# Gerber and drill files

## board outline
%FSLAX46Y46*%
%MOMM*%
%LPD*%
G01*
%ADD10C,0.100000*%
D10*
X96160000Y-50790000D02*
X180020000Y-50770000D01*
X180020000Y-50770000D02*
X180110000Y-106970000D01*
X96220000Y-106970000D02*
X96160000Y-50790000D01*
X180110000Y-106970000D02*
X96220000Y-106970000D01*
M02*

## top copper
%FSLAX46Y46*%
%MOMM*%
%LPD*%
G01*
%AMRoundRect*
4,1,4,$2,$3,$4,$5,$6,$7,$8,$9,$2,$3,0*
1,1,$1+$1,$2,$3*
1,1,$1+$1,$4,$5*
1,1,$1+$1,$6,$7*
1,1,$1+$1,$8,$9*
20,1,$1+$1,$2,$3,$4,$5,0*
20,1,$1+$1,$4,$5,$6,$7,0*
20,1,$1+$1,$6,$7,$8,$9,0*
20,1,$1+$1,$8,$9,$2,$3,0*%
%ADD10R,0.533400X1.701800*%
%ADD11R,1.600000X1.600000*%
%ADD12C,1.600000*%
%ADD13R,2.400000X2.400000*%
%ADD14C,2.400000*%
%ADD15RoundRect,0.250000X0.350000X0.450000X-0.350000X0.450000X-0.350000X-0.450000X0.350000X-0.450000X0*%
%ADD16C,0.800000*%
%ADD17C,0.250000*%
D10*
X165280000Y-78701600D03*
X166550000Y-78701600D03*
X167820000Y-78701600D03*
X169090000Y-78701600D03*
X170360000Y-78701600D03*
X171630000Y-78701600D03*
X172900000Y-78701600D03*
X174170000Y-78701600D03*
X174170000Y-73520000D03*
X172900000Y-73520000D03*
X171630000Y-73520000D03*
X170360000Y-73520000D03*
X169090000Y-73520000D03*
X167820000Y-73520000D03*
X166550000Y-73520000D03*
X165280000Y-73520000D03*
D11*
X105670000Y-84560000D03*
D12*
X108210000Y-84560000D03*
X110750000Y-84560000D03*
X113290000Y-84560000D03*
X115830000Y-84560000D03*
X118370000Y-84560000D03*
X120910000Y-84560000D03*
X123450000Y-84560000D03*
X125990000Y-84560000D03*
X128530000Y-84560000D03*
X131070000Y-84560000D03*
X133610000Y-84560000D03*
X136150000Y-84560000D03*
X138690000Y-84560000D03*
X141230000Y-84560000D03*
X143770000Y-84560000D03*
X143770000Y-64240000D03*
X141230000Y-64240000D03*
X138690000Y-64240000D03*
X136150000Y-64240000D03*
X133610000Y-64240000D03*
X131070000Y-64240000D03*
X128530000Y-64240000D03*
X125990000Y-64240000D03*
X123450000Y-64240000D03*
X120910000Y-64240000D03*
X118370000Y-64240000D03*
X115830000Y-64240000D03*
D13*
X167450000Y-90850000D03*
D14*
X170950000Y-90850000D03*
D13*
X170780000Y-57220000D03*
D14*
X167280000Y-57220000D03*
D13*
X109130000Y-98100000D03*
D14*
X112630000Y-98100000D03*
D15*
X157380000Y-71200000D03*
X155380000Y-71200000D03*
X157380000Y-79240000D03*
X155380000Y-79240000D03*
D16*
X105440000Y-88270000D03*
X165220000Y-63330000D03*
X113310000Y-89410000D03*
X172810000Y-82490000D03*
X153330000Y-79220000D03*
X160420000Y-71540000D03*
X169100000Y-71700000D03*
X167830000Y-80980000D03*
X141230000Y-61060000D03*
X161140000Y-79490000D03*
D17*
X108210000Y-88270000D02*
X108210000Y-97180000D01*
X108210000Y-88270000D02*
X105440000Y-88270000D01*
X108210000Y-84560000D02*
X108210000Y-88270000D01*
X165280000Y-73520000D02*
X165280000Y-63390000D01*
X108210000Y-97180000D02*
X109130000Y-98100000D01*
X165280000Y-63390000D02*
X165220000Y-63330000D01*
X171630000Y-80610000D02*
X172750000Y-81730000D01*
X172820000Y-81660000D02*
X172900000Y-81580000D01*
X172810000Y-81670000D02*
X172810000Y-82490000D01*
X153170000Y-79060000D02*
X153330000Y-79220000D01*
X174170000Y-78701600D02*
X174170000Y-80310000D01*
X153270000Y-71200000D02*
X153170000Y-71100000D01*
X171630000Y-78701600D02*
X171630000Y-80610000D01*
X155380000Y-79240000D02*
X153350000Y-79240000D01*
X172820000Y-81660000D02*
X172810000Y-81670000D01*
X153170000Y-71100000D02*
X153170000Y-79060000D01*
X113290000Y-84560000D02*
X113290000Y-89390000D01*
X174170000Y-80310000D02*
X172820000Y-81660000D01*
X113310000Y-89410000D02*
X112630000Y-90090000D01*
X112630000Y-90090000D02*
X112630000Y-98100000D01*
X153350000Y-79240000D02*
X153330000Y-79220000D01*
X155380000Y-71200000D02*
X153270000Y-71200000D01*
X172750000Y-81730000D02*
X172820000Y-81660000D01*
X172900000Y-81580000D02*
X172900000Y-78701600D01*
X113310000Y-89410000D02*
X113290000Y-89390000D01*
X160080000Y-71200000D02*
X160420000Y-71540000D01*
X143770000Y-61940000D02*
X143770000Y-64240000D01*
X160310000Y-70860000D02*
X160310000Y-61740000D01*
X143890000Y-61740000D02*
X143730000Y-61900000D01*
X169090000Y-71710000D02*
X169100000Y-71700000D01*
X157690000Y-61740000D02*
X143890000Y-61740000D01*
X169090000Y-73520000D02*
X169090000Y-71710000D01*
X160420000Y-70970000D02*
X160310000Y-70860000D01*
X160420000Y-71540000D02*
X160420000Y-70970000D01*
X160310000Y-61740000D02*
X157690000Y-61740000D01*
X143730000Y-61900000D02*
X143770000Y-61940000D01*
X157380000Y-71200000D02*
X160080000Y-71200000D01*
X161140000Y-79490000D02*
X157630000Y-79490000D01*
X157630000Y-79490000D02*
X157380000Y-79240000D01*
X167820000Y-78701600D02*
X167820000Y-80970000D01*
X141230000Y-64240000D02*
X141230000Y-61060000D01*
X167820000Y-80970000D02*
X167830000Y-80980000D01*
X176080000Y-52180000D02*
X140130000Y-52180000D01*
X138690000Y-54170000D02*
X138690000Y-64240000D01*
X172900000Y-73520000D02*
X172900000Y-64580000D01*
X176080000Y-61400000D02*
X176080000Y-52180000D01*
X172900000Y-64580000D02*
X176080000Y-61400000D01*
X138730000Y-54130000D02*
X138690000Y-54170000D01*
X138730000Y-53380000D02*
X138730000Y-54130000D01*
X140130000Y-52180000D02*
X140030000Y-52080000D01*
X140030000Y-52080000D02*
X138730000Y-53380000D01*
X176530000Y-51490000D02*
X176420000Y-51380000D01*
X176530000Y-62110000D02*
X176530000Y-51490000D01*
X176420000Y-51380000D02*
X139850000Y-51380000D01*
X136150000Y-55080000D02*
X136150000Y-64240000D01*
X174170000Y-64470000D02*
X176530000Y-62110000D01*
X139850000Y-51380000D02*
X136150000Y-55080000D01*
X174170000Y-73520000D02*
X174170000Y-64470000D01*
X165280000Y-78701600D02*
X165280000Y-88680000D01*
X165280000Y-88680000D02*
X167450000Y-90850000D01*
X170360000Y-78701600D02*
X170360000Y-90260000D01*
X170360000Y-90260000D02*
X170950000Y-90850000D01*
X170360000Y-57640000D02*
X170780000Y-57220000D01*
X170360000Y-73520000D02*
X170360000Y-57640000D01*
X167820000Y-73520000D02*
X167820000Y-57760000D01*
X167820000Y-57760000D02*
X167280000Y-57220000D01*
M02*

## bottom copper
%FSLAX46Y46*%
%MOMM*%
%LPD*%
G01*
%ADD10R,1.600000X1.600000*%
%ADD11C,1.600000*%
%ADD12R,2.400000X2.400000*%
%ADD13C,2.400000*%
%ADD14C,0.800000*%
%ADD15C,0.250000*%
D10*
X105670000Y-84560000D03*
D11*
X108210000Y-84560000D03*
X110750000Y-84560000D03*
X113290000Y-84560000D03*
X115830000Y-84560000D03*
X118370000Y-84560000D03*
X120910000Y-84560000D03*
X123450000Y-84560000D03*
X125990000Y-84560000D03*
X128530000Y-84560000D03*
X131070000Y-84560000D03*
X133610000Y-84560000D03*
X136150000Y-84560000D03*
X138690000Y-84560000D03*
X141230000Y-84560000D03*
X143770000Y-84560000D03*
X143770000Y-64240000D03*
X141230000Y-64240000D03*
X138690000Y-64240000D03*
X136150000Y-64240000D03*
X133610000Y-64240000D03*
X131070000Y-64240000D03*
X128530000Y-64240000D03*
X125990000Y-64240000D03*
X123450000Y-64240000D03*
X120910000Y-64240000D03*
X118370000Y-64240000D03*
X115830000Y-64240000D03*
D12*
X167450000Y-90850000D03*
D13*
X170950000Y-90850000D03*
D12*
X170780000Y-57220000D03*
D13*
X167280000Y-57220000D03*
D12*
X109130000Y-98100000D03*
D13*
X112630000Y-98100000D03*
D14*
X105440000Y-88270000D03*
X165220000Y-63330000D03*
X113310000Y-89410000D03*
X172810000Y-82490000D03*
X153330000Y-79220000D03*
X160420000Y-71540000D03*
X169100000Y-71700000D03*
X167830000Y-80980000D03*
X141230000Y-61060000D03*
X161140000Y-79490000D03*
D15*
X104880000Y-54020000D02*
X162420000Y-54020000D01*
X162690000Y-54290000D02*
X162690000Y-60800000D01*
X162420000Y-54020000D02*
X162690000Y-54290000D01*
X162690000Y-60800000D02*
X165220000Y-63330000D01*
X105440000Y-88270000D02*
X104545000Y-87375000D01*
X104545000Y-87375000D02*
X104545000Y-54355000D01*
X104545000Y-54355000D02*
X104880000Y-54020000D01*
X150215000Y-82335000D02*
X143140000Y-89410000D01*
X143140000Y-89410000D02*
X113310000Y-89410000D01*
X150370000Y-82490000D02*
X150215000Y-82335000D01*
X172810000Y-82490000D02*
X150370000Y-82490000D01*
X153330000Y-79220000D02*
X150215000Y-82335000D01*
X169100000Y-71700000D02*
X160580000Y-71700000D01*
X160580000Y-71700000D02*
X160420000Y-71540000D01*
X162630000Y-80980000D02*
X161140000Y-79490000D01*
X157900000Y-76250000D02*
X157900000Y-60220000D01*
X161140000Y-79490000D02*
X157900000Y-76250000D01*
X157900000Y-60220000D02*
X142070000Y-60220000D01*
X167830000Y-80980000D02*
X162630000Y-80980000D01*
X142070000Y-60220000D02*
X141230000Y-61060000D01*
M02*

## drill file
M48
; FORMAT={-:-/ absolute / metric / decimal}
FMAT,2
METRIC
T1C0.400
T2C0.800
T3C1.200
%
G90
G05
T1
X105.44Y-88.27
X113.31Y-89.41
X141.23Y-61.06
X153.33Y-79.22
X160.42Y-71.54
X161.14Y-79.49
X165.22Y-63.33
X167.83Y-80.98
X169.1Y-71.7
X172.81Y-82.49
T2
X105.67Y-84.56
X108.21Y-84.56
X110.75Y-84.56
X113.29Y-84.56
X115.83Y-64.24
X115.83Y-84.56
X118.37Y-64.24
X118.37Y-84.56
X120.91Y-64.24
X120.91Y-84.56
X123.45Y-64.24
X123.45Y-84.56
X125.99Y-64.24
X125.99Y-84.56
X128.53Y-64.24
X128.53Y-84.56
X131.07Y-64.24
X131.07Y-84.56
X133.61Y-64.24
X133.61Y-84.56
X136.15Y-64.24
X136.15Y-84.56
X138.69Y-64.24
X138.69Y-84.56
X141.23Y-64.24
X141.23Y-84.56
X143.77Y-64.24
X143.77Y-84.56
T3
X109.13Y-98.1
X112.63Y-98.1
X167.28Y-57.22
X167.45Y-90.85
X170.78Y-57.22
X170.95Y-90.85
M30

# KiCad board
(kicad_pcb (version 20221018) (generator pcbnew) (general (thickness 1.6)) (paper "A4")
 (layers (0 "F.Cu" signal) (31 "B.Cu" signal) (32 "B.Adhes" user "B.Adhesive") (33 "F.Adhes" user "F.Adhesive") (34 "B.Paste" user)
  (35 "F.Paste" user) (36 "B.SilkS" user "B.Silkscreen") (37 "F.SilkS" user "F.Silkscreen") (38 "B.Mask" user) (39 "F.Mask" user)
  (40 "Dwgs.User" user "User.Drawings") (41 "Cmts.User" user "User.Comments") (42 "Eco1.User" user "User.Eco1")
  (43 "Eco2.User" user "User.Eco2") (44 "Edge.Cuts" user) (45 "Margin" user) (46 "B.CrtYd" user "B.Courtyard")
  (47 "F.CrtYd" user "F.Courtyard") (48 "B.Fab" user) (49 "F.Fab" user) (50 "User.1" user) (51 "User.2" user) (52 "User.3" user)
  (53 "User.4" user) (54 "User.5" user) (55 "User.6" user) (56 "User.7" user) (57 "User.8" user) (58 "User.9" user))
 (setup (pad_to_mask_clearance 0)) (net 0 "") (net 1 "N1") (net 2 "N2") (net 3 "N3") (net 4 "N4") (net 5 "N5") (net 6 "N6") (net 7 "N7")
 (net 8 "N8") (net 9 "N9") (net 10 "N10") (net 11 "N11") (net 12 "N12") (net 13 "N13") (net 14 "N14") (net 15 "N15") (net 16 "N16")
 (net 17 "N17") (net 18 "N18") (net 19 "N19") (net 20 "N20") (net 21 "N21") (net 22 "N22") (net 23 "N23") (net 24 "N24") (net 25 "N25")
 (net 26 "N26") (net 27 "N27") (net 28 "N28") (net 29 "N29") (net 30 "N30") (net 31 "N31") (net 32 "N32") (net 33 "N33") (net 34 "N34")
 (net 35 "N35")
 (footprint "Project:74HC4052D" (layer "F.Cu") (at 169.725 76.1108 90)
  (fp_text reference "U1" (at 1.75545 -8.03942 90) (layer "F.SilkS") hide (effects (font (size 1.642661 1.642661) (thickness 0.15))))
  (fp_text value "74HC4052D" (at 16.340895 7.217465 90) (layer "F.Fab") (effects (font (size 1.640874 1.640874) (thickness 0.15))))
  (pad "1" smd rect (at -2.5908 -4.445 90) (size 1.7018 0.5334) (layers "F.Cu" "F.Paste" "F.Mask") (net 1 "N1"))
  (pad "2" smd rect (at -2.5908 -3.175 90) (size 1.7018 0.5334) (layers "F.Cu" "F.Paste" "F.Mask") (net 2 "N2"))
  (pad "3" smd rect (at -2.5908 -1.905 90) (size 1.7018 0.5334) (layers "F.Cu" "F.Paste" "F.Mask") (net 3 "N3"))
  (pad "4" smd rect (at -2.5908 -0.635 90) (size 1.7018 0.5334) (layers "F.Cu" "F.Paste" "F.Mask") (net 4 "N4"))
  (pad "5" smd rect (at -2.5908 0.635 90) (size 1.7018 0.5334) (layers "F.Cu" "F.Paste" "F.Mask") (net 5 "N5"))
  (pad "6" smd rect (at -2.5908 1.905 90) (size 1.7018 0.5334) (layers "F.Cu" "F.Paste" "F.Mask") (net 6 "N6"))
  (pad "7" smd rect (at -2.5908 3.175 90) (size 1.7018 0.5334) (layers "F.Cu" "F.Paste" "F.Mask") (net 6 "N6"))
  (pad "8" smd rect (at -2.5908 4.445 90) (size 1.7018 0.5334) (layers "F.Cu" "F.Paste" "F.Mask") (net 6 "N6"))
  (pad "9" smd rect (at 2.5908 4.445 90) (size 1.7018 0.5334) (layers "F.Cu" "F.Paste" "F.Mask") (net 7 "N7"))
  (pad "10" smd rect (at 2.5908 3.175 90) (size 1.7018 0.5334) (layers "F.Cu" "F.Paste" "F.Mask") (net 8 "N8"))
  (pad "11" smd rect (at 2.5908 1.905 90) (size 1.7018 0.5334) (layers "F.Cu" "F.Paste" "F.Mask") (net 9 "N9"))
  (pad "12" smd rect (at 2.5908 0.635 90) (size 1.7018 0.5334) (layers "F.Cu" "F.Paste" "F.Mask") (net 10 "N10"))
  (pad "13" smd rect (at 2.5908 -0.635 90) (size 1.7018 0.5334) (layers "F.Cu" "F.Paste" "F.Mask") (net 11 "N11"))
  (pad "14" smd rect (at 2.5908 -1.905 90) (size 1.7018 0.5334) (layers "F.Cu" "F.Paste" "F.Mask") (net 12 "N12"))
  (pad "15" smd rect (at 2.5908 -3.175 90) (size 1.7018 0.5334) (layers "F.Cu" "F.Paste" "F.Mask") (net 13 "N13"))
  (pad "16" smd rect (at 2.5908 -4.445 90) (size 1.7018 0.5334) (layers "F.Cu" "F.Paste" "F.Mask") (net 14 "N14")))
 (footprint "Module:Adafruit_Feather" (layer "F.Cu") (at 105.67 84.56 90)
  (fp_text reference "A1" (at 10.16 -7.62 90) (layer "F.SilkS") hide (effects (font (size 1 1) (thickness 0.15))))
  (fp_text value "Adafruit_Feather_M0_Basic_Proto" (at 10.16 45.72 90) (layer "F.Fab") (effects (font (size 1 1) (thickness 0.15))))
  (pad "1" thru_hole rect (at 0 0 270) (size 1.6 1.6) (drill 0.8) (layers "*.Cu" "*.Mask") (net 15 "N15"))
  (pad "2" thru_hole circle (at 0 2.54 270) (size 1.6 1.6) (drill 0.8) (layers "*.Cu" "*.Mask") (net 14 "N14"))
  (pad "3" thru_hole circle (at 0 5.08 270) (size 1.6 1.6) (drill 0.8) (layers "*.Cu" "*.Mask") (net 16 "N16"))
  (pad "4" thru_hole circle (at 0 7.62 270) (size 1.6 1.6) (drill 0.8) (layers "*.Cu" "*.Mask") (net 6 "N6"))
  (pad "5" thru_hole circle (at 0 10.16 270) (size 1.6 1.6) (drill 0.8) (layers "*.Cu" "*.Mask") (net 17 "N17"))
  (pad "6" thru_hole circle (at 0 12.7 270) (size 1.6 1.6) (drill 0.8) (layers "*.Cu" "*.Mask") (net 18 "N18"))
  (pad "7" thru_hole circle (at 0 15.24 270) (size 1.6 1.6) (drill 0.8) (layers "*.Cu" "*.Mask") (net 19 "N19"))
  (pad "8" thru_hole circle (at 0 17.78 270) (size 1.6 1.6) (drill 0.8) (layers "*.Cu" "*.Mask") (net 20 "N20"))
  (pad "9" thru_hole circle (at 0 20.32 270) (size 1.6 1.6) (drill 0.8) (layers "*.Cu" "*.Mask") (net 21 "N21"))
  (pad "10" thru_hole circle (at 0 22.86 270) (size 1.6 1.6) (drill 0.8) (layers "*.Cu" "*.Mask") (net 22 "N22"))
  (pad "11" thru_hole circle (at 0 25.4 270) (size 1.6 1.6) (drill 0.8) (layers "*.Cu" "*.Mask") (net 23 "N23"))
  (pad "12" thru_hole circle (at 0 27.94 270) (size 1.6 1.6) (drill 0.8) (layers "*.Cu" "*.Mask") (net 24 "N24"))
  (pad "13" thru_hole circle (at 0 30.48 270) (size 1.6 1.6) (drill 0.8) (layers "*.Cu" "*.Mask") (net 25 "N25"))
  (pad "14" thru_hole circle (at 0 33.02 270) (size 1.6 1.6) (drill 0.8) (layers "*.Cu" "*.Mask") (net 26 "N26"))
  (pad "15" thru_hole circle (at 0 35.56 270) (size 1.6 1.6) (drill 0.8) (layers "*.Cu" "*.Mask") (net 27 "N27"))
  (pad "16" thru_hole circle (at 0 38.1 270) (size 1.6 1.6) (drill 0.8) (layers "*.Cu" "*.Mask") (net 6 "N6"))
  (pad "17" thru_hole circle (at 20.32 38.1 270) (size 1.6 1.6) (drill 0.8) (layers "*.Cu" "*.Mask") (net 11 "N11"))
  (pad "18" thru_hole circle (at 20.32 35.56 270) (size 1.6 1.6) (drill 0.8) (layers "*.Cu" "*.Mask") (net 3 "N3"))
  (pad "19" thru_hole circle (at 20.32 33.02 270) (size 1.6 1.6) (drill 0.8) (layers "*.Cu" "*.Mask") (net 8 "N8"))
  (pad "20" thru_hole circle (at 20.32 30.48 270) (size 1.6 1.6) (drill 0.8) (layers "*.Cu" "*.Mask") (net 7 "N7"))
  (pad "21" thru_hole circle (at 20.32 27.94 270) (size 1.6 1.6) (drill 0.8) (layers "*.Cu" "*.Mask") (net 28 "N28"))
  (pad "22" thru_hole circle (at 20.32 25.4 270) (size 1.6 1.6) (drill 0.8) (layers "*.Cu" "*.Mask") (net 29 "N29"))
  (pad "23" thru_hole circle (at 20.32 22.86 270) (size 1.6 1.6) (drill 0.8) (layers "*.Cu" "*.Mask") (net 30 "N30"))
  (pad "24" thru_hole circle (at 20.32 20.32 270) (size 1.6 1.6) (drill 0.8) (layers "*.Cu" "*.Mask") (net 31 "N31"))
  (pad "25" thru_hole circle (at 20.32 17.78 270) (size 1.6 1.6) (drill 0.8) (layers "*.Cu" "*.Mask") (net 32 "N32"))
  (pad "26" thru_hole circle (at 20.32 15.24 270) (size 1.6 1.6) (drill 0.8) (layers "*.Cu" "*.Mask") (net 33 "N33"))
  (pad "27" thru_hole circle (at 20.32 12.7 270) (size 1.6 1.6) (drill 0.8) (layers "*.Cu" "*.Mask") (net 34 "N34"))
  (pad "28" thru_hole circle (at 20.32 10.16 270) (size 1.6 1.6) (drill 0.8) (layers "*.Cu" "*.Mask") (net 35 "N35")))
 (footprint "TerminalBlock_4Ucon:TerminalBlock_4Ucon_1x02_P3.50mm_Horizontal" (layer "F.Cu") (at 167.45 90.85)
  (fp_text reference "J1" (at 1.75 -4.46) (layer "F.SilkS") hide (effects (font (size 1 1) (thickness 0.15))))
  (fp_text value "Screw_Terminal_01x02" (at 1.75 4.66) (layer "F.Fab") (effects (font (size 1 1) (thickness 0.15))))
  (pad "1" thru_hole rect (at 0 0) (size 2.4 2.4) (drill 1.2) (layers "*.Cu" "*.Mask") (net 1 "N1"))
  (pad "2" thru_hole circle (at 3.5 0) (size 2.4 2.4) (drill 1.2) (layers "*.Cu" "*.Mask") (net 5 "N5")))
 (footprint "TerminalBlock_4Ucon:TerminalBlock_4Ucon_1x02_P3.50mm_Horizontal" (layer "F.Cu") (at 170.78 57.22 180)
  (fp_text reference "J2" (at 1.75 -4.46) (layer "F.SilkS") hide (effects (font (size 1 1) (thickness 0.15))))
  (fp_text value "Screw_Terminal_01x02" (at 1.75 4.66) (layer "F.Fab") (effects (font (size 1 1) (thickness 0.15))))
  (pad "1" thru_hole rect (at 0 0 180) (size 2.4 2.4) (drill 1.2) (layers "*.Cu" "*.Mask") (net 10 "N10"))
  (pad "2" thru_hole circle (at 3.5 0 180) (size 2.4 2.4) (drill 1.2) (layers "*.Cu" "*.Mask") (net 12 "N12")))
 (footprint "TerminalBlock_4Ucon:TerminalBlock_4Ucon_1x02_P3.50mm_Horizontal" (layer "F.Cu") (at 109.13 98.1)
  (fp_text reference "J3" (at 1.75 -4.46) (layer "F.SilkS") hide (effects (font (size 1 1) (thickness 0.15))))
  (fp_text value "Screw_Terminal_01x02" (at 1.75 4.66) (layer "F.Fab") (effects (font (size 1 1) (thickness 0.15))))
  (pad "1" thru_hole rect (at 0 0) (size 2.4 2.4) (drill 1.2) (layers "*.Cu" "*.Mask") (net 14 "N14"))
  (pad "2" thru_hole circle (at 3.5 0) (size 2.4 2.4) (drill 1.2) (layers "*.Cu" "*.Mask") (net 6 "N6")))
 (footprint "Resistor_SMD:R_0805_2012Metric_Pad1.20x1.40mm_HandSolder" (layer "F.Cu") (at 156.38 71.2 180)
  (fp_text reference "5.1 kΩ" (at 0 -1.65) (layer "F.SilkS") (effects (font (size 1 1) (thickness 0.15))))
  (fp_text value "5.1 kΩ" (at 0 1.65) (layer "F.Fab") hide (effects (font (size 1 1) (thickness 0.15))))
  (pad "1" smd roundrect (at -1 0 180) (size 1.2 1.4) (layers "F.Cu" "F.Paste" "F.Mask") (roundrect_rratio 0.208333) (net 11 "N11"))
  (pad "2" smd roundrect (at 1 0 180) (size 1.2 1.4) (layers "F.Cu" "F.Paste" "F.Mask") (roundrect_rratio 0.208333) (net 6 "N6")))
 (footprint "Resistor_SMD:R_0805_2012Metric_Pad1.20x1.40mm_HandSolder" (layer "F.Cu") (at 156.38 79.24 180)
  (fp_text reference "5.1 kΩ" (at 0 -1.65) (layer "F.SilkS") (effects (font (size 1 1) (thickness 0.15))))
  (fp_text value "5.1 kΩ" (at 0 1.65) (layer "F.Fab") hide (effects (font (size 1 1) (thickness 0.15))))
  (pad "1" smd roundrect (at -1 0 180) (size 1.2 1.4) (layers "F.Cu" "F.Paste" "F.Mask") (roundrect_rratio 0.208333) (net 3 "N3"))
  (pad "2" smd roundrect (at 1 0 180) (size 1.2 1.4) (layers "F.Cu" "F.Paste" "F.Mask") (roundrect_rratio 0.208333) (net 6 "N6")))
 (gr_line (start 96.16 50.79) (end 180.02 50.77) (stroke (width 0.1) (type default)) (layer "Edge.Cuts"))
 (gr_line (start 180.02 50.77) (end 180.11 106.97) (stroke (width 0.1) (type default)) (layer "Edge.Cuts"))
 (gr_line (start 96.22 106.97) (end 96.16 50.79) (stroke (width 0.1) (type default)) (layer "Edge.Cuts"))
 (gr_line (start 180.11 106.97) (end 96.22 106.97) (stroke (width 0.1) (type default)) (layer "Edge.Cuts"))
 (segment (start 108.21 88.27) (end 108.21 97.18) (width 0.25) (layer "F.Cu") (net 14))
 (segment (start 108.21 88.27) (end 105.44 88.27) (width 0.25) (layer "F.Cu") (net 14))
 (segment (start 108.21 84.56) (end 108.21 88.27) (width 0.25) (layer "F.Cu") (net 14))
 (segment (start 165.28 73.52) (end 165.28 63.39) (width 0.25) (layer "F.Cu") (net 14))
 (segment (start 108.21 97.18) (end 109.13 98.1) (width 0.25) (layer "F.Cu") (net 14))
 (segment (start 165.28 63.39) (end 165.22 63.33) (width 0.25) (layer "F.Cu") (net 14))
 (via (at 105.44 88.27) (size 0.8) (drill 0.4) (layers "F.Cu" "B.Cu") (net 14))
 (via (at 165.22 63.33) (size 0.8) (drill 0.4) (layers "F.Cu" "B.Cu") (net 14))
 (segment (start 104.88 54.02) (end 162.42 54.02) (width 0.25) (layer "B.Cu") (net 14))
 (segment (start 162.69 54.29) (end 162.69 60.8) (width 0.25) (layer "B.Cu") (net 14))
 (segment (start 162.42 54.02) (end 162.69 54.29) (width 0.25) (layer "B.Cu") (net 14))
 (segment (start 162.69 60.8) (end 165.22 63.33) (width 0.25) (layer "B.Cu") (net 14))
 (segment (start 105.44 88.27) (end 104.545 87.375) (width 0.25) (layer "B.Cu") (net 14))
 (segment (start 104.545 87.375) (end 104.545 54.355) (width 0.25) (layer "B.Cu") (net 14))
 (segment (start 104.545 54.355) (end 104.88 54.02) (width 0.25) (layer "B.Cu") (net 14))
 (segment (start 171.63 80.61) (end 172.75 81.73) (width 0.25) (layer "F.Cu") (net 6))
 (segment (start 172.82 81.66) (end 172.9 81.58) (width 0.25) (layer "F.Cu") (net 6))
 (segment (start 172.81 81.67) (end 172.81 82.49) (width 0.25) (layer "F.Cu") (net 6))
 (segment (start 153.17 79.06) (end 153.33 79.22) (width 0.25) (layer "F.Cu") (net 6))
 (segment (start 174.17 78.7016) (end 174.17 80.31) (width 0.25) (layer "F.Cu") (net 6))
 (segment (start 153.27 71.2) (end 153.17 71.1) (width 0.25) (layer "F.Cu") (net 6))
 (segment (start 171.63 78.7016) (end 171.63 80.61) (width 0.25) (layer "F.Cu") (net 6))
 (segment (start 155.38 79.24) (end 153.35 79.24) (width 0.25) (layer "F.Cu") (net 6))
 (segment (start 172.82 81.66) (end 172.81 81.67) (width 0.25) (layer "F.Cu") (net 6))
 (segment (start 153.17 71.1) (end 153.17 79.06) (width 0.25) (layer "F.Cu") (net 6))
 (segment (start 113.29 84.56) (end 113.29 89.39) (width 0.25) (layer "F.Cu") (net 6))
 (segment (start 174.17 80.31) (end 172.82 81.66) (width 0.25) (layer "F.Cu") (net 6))
 (segment (start 113.31 89.41) (end 112.63 90.09) (width 0.25) (layer "F.Cu") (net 6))
 (segment (start 112.63 90.09) (end 112.63 98.1) (width 0.25) (layer "F.Cu") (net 6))
 (segment (start 153.35 79.24) (end 153.33 79.22) (width 0.25) (layer "F.Cu") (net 6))
 (segment (start 155.38 71.2) (end 153.27 71.2) (width 0.25) (layer "F.Cu") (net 6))
 (segment (start 172.75 81.73) (end 172.82 81.66) (width 0.25) (layer "F.Cu") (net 6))
 (segment (start 172.9 81.58) (end 172.9 78.7016) (width 0.25) (layer "F.Cu") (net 6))
 (segment (start 113.31 89.41) (end 113.29 89.39) (width 0.25) (layer "F.Cu") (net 6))
 (via (at 113.31 89.41) (size 0.8) (drill 0.4) (layers "F.Cu" "B.Cu") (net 6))
 (via (at 172.81 82.49) (size 0.8) (drill 0.4) (layers "F.Cu" "B.Cu") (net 6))
 (via (at 153.33 79.22) (size 0.8) (drill 0.4) (layers "F.Cu" "B.Cu") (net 6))
 (segment (start 150.215 82.335) (end 143.14 89.41) (width 0.25) (layer "B.Cu") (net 6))
 (segment (start 143.14 89.41) (end 113.31 89.41) (width 0.25) (layer "B.Cu") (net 6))
 (segment (start 150.37 82.49) (end 150.215 82.335) (width 0.25) (layer "B.Cu") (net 6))
 (segment (start 172.81 82.49) (end 150.37 82.49) (width 0.25) (layer "B.Cu") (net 6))
 (segment (start 153.33 79.22) (end 150.215 82.335) (width 0.25) (layer "B.Cu") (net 6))
 (segment (start 160.08 71.2) (end 160.42 71.54) (width 0.25) (layer "F.Cu") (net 11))
 (segment (start 143.77 61.94) (end 143.77 64.24) (width 0.25) (layer "F.Cu") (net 11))
 (segment (start 160.31 70.86) (end 160.31 61.74) (width 0.25) (layer "F.Cu") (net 11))
 (segment (start 143.89 61.74) (end 143.73 61.9) (width 0.25) (layer "F.Cu") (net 11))
 (segment (start 169.09 71.71) (end 169.1 71.7) (width 0.25) (layer "F.Cu") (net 11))
 (segment (start 157.69 61.74) (end 143.89 61.74) (width 0.25) (layer "F.Cu") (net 11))
 (segment (start 169.09 73.52) (end 169.09 71.71) (width 0.25) (layer "F.Cu") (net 11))
 (segment (start 160.42 70.97) (end 160.31 70.86) (width 0.25) (layer "F.Cu") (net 11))
 (segment (start 160.42 71.54) (end 160.42 70.97) (width 0.25) (layer "F.Cu") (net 11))
 (segment (start 160.31 61.74) (end 157.69 61.74) (width 0.25) (layer "F.Cu") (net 11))
 (segment (start 143.73 61.9) (end 143.77 61.94) (width 0.25) (layer "F.Cu") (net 11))
 (segment (start 157.38 71.2) (end 160.08 71.2) (width 0.25) (layer "F.Cu") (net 11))
 (via (at 160.42 71.54) (size 0.8) (drill 0.4) (layers "F.Cu" "B.Cu") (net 11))
 (via (at 169.1 71.7) (size 0.8) (drill 0.4) (layers "F.Cu" "B.Cu") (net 11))
 (segment (start 169.1 71.7) (end 160.58 71.7) (width 0.25) (layer "B.Cu") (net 11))
 (segment (start 160.58 71.7) (end 160.42 71.54) (width 0.25) (layer "B.Cu") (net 11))
 (segment (start 161.14 79.49) (end 157.63 79.49) (width 0.25) (layer "F.Cu") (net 3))
 (segment (start 157.63 79.49) (end 157.38 79.24) (width 0.25) (layer "F.Cu") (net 3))
 (segment (start 167.82 78.7016) (end 167.82 80.97) (width 0.25) (layer "F.Cu") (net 3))
 (segment (start 141.23 64.24) (end 141.23 61.06) (width 0.25) (layer "F.Cu") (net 3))
 (segment (start 167.82 80.97) (end 167.83 80.98) (width 0.25) (layer "F.Cu") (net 3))
 (via (at 167.83 80.98) (size 0.8) (drill 0.4) (layers "F.Cu" "B.Cu") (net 3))
 (via (at 141.23 61.06) (size 0.8) (drill 0.4) (layers "F.Cu" "B.Cu") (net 3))
 (via (at 161.14 79.49) (size 0.8) (drill 0.4) (layers "F.Cu" "B.Cu") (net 3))
 (segment (start 162.63 80.98) (end 161.14 79.49) (width 0.25) (layer "B.Cu") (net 3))
 (segment (start 157.9 76.25) (end 157.9 60.22) (width 0.25) (layer "B.Cu") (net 3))
 (segment (start 161.14 79.49) (end 157.9 76.25) (width 0.25) (layer "B.Cu") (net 3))
 (segment (start 157.9 60.22) (end 142.07 60.22) (width 0.25) (layer "B.Cu") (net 3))
 (segment (start 167.83 80.98) (end 162.63 80.98) (width 0.25) (layer "B.Cu") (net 3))
 (segment (start 142.07 60.22) (end 141.23 61.06) (width 0.25) (layer "B.Cu") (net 3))
 (segment (start 176.08 52.18) (end 140.13 52.18) (width 0.25) (layer "F.Cu") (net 8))
 (segment (start 138.69 54.17) (end 138.69 64.24) (width 0.25) (layer "F.Cu") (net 8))
 (segment (start 172.9 73.52) (end 172.9 64.58) (width 0.25) (layer "F.Cu") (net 8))
 (segment (start 176.08 61.4) (end 176.08 52.18) (width 0.25) (layer "F.Cu") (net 8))
 (segment (start 172.9 64.58) (end 176.08 61.4) (width 0.25) (layer "F.Cu") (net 8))
 (segment (start 138.73 54.13) (end 138.69 54.17) (width 0.25) (layer "F.Cu") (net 8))
 (segment (start 138.73 53.38) (end 138.73 54.13) (width 0.25) (layer "F.Cu") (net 8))
 (segment (start 140.13 52.18) (end 140.03 52.08) (width 0.25) (layer "F.Cu") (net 8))
 (segment (start 140.03 52.08) (end 138.73 53.38) (width 0.25) (layer "F.Cu") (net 8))
 (segment (start 176.53 51.49) (end 176.42 51.38) (width 0.25) (layer "F.Cu") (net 7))
 (segment (start 176.53 62.11) (end 176.53 51.49) (width 0.25) (layer "F.Cu") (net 7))
 (segment (start 176.42 51.38) (end 139.85 51.38) (width 0.25) (layer "F.Cu") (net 7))
 (segment (start 136.15 55.08) (end 136.15 64.24) (width 0.25) (layer "F.Cu") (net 7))
 (segment (start 174.17 64.47) (end 176.53 62.11) (width 0.25) (layer "F.Cu") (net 7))
 (segment (start 139.85 51.38) (end 136.15 55.08) (width 0.25) (layer "F.Cu") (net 7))
 (segment (start 174.17 73.52) (end 174.17 64.47) (width 0.25) (layer "F.Cu") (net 7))
 (segment (start 165.28 78.7016) (end 165.28 88.68) (width 0.25) (layer "F.Cu") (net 1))
 (segment (start 165.28 88.68) (end 167.45 90.85) (width 0.25) (layer "F.Cu") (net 1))
 (segment (start 170.36 78.7016) (end 170.36 90.26) (width 0.25) (layer "F.Cu") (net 5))
 (segment (start 170.36 90.26) (end 170.95 90.85) (width 0.25) (layer "F.Cu") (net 5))
 (segment (start 170.36 57.64) (end 170.78 57.22) (width 0.25) (layer "F.Cu") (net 10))
 (segment (start 170.36 73.52) (end 170.36 57.64) (width 0.25) (layer "F.Cu") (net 10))
 (segment (start 167.82 73.52) (end 167.82 57.76) (width 0.25) (layer "F.Cu") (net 12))
 (segment (start 167.82 57.76) (end 167.28 57.22) (width 0.25) (layer "F.Cu") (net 12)))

